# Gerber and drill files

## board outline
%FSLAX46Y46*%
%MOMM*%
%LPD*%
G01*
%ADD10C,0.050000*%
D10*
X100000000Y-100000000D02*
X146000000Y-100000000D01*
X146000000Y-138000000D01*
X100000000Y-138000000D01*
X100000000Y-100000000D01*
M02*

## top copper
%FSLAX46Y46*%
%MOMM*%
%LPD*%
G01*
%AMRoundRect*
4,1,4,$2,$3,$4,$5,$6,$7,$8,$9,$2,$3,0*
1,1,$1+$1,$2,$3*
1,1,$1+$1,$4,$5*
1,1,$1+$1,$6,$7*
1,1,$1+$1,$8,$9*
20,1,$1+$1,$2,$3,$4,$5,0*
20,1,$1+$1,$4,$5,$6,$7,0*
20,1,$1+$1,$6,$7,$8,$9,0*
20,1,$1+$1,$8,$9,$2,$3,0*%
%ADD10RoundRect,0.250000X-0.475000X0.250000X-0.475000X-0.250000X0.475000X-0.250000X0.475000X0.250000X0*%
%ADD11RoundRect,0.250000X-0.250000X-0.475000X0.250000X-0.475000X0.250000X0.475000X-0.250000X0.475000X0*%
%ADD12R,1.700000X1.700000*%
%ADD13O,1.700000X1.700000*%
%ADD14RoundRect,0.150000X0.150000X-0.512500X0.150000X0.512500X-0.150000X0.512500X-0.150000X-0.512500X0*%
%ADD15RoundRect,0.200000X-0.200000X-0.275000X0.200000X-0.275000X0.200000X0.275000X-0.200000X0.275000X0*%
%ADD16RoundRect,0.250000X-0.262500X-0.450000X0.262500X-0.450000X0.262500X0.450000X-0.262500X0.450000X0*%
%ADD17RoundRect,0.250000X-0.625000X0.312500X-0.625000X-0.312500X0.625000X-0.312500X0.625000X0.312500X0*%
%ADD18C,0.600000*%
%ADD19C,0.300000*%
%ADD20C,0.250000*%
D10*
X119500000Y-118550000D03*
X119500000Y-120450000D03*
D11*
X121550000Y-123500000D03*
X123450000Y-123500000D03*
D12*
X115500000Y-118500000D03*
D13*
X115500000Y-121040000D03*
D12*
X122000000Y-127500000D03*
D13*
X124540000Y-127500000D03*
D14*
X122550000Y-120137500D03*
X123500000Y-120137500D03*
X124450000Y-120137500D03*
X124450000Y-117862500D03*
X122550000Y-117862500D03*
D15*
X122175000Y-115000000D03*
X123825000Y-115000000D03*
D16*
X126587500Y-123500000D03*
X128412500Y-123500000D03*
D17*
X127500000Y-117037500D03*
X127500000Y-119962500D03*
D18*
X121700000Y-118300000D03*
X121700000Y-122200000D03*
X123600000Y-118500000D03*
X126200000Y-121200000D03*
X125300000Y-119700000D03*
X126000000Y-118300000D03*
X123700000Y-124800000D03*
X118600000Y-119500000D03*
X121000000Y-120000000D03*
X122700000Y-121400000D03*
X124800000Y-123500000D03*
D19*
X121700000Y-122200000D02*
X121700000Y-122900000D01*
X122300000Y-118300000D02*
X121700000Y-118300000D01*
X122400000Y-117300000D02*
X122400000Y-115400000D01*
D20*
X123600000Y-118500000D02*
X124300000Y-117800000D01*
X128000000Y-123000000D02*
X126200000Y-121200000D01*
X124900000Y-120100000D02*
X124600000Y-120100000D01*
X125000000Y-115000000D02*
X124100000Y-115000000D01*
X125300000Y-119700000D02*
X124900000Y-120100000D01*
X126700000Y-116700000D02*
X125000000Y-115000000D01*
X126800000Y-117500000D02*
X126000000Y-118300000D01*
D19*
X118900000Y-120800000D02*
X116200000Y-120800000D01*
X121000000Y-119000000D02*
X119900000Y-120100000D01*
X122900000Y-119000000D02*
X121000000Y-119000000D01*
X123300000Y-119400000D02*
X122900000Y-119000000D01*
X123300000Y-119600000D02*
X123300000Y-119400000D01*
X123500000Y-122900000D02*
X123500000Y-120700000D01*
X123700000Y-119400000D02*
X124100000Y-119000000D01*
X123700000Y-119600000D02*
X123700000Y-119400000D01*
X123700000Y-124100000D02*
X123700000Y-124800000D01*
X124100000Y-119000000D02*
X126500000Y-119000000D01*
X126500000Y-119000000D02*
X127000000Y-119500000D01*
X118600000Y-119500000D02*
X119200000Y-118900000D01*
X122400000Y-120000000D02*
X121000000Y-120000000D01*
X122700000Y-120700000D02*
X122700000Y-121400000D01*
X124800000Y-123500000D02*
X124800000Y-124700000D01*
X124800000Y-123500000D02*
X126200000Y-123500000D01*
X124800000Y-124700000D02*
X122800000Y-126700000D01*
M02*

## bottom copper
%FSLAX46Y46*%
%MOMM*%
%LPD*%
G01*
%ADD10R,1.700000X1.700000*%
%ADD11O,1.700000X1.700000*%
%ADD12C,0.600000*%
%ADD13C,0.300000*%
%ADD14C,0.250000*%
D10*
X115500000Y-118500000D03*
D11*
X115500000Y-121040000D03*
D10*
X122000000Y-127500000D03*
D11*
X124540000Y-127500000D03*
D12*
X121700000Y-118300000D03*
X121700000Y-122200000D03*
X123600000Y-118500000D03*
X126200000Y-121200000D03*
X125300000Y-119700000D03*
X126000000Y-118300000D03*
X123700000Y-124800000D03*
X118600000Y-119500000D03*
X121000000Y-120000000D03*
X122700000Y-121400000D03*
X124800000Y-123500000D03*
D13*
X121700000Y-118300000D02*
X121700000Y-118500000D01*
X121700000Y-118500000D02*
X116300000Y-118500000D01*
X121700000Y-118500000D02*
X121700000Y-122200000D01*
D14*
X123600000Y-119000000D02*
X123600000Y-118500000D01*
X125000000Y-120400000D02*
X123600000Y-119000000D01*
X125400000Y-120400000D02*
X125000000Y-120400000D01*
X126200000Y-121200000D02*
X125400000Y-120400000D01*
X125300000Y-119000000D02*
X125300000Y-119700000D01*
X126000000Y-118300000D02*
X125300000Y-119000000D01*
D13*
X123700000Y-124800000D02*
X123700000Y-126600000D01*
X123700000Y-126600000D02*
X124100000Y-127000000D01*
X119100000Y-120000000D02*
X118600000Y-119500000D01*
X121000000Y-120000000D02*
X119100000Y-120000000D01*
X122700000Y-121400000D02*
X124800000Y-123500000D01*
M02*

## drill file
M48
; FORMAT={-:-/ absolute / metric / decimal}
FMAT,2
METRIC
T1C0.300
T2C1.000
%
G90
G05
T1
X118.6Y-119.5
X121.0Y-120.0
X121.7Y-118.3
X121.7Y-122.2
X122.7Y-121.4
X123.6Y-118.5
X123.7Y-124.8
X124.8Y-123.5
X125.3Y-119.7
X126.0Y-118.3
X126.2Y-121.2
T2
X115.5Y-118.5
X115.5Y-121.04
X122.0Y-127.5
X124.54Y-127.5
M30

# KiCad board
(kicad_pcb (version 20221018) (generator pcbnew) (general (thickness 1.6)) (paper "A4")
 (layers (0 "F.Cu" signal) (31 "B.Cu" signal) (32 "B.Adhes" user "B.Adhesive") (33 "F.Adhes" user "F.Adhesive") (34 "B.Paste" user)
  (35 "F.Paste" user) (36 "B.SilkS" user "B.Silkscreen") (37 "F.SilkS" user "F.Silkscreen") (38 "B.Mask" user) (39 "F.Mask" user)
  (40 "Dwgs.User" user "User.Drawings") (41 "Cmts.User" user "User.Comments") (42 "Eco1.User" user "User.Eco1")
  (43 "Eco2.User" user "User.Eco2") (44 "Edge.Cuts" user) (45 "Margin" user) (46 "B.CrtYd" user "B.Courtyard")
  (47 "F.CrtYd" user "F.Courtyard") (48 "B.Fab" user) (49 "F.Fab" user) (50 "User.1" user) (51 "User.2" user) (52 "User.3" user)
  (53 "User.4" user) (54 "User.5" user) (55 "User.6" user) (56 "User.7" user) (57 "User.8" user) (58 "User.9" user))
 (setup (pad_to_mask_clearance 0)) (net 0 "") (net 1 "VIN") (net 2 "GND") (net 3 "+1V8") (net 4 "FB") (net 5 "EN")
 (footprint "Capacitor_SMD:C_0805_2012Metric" (layer "F.Cu") (at 119.5 119.5 -90)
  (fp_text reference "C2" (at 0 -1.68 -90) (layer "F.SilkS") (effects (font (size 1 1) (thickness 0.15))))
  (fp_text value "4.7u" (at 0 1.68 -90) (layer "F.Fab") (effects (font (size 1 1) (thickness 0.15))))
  (pad "1" smd roundrect (at -0.95 0 270) (size 1 1.45) (layers "F.Cu" "F.Paste" "F.Mask") (roundrect_rratio 0.25) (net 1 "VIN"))
  (pad "2" smd roundrect (at 0.95 0 270) (size 1 1.45) (layers "F.Cu" "F.Paste" "F.Mask") (roundrect_rratio 0.25) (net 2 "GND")))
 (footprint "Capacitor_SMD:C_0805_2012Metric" (layer "F.Cu") (at 122.5 123.5)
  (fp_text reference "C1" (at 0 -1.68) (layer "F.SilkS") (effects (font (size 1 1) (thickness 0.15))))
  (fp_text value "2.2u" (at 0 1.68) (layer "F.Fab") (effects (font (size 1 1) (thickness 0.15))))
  (pad "1" smd roundrect (at -0.95 0) (size 1 1.45) (layers "F.Cu" "F.Paste" "F.Mask") (roundrect_rratio 0.25) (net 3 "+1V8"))
  (pad "2" smd roundrect (at 0.95 0) (size 1 1.45) (layers "F.Cu" "F.Paste" "F.Mask") (roundrect_rratio 0.25) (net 2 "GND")))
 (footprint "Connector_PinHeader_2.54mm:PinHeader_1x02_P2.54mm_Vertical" (layer "F.Cu") (at 115.5 118.5)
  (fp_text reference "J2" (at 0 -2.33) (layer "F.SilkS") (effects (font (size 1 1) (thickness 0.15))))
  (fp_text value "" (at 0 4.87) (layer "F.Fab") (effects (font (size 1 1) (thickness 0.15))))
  (pad "1" thru_hole rect (at 0 0) (size 1.7 1.7) (drill 1) (layers "*.Cu" "*.Mask") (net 3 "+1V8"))
  (pad "2" thru_hole oval (at 0 2.54) (size 1.7 1.7) (drill 1) (layers "*.Cu" "*.Mask") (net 2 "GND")))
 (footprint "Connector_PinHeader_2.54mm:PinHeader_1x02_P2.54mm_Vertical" (layer "F.Cu") (at 122 127.5 90)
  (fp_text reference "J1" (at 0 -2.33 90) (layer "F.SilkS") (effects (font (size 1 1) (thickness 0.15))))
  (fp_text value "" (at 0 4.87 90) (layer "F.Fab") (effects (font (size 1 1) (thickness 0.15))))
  (pad "1" thru_hole rect (at 0 0 90) (size 1.7 1.7) (drill 1) (layers "*.Cu" "*.Mask") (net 1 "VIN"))
  (pad "2" thru_hole oval (at 0 2.54 90) (size 1.7 1.7) (drill 1) (layers "*.Cu" "*.Mask") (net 2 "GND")))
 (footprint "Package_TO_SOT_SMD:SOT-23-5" (layer "F.Cu") (at 123.5 119 90)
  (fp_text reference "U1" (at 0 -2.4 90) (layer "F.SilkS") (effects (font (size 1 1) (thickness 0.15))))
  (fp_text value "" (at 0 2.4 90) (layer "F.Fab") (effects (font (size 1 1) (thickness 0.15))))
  (pad "1" smd roundrect (at -1.1375 -0.95 90) (size 1.325 0.6) (layers "F.Cu" "F.Paste" "F.Mask") (roundrect_rratio 0.25) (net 1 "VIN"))
  (pad "2" smd roundrect (at -1.1375 0 90) (size 1.325 0.6) (layers "F.Cu" "F.Paste" "F.Mask") (roundrect_rratio 0.25) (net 2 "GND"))
  (pad "3" smd roundrect (at -1.1375 0.95 90) (size 1.325 0.6) (layers "F.Cu" "F.Paste" "F.Mask") (roundrect_rratio 0.25) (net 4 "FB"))
  (pad "4" smd roundrect (at 1.1375 0.95 90) (size 1.325 0.6) (layers "F.Cu" "F.Paste" "F.Mask") (roundrect_rratio 0.25) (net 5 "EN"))
  (pad "5" smd roundrect (at 1.1375 -0.95 90) (size 1.325 0.6) (layers "F.Cu" "F.Paste" "F.Mask") (roundrect_rratio 0.25) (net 3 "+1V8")))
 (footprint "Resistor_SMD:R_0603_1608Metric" (layer "F.Cu") (at 123 115)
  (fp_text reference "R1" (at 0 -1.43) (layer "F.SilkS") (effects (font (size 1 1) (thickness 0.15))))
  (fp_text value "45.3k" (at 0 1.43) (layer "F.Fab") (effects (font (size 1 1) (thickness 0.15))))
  (pad "1" smd roundrect (at -0.825 0) (size 0.8 0.95) (layers "F.Cu" "F.Paste" "F.Mask") (roundrect_rratio 0.25) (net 3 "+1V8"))
  (pad "2" smd roundrect (at 0.825 0) (size 0.8 0.95) (layers "F.Cu" "F.Paste" "F.Mask") (roundrect_rratio 0.25) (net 4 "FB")))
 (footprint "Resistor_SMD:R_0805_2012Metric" (layer "F.Cu") (at 127.5 123.5)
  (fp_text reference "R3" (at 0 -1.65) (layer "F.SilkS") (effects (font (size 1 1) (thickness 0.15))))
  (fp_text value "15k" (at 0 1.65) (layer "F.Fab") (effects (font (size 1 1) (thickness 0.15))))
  (pad "1" smd roundrect (at -0.9125 0) (size 1.025 1.4) (layers "F.Cu" "F.Paste" "F.Mask") (roundrect_rratio 0.243902) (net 1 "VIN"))
  (pad "2" smd roundrect (at 0.9125 0) (size 1.025 1.4) (layers "F.Cu" "F.Paste" "F.Mask") (roundrect_rratio 0.243902) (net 5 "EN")))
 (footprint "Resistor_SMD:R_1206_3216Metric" (layer "F.Cu") (at 127.5 118.5 -90)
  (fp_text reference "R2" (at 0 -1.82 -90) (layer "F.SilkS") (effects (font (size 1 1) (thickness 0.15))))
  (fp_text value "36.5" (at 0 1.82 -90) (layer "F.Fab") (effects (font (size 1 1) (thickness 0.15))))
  (pad "1" smd roundrect (at -1.4625 0 270) (size 1.125 1.75) (layers "F.Cu" "F.Paste" "F.Mask") (roundrect_rratio 0.222222) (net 4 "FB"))
  (pad "2" smd roundrect (at 1.4625 0 270) (size 1.125 1.75) (layers "F.Cu" "F.Paste" "F.Mask") (roundrect_rratio 0.222222) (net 2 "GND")))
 (gr_rect (start 100 100) (end 146 138) (stroke (width 0.05) (type default)) (fill none) (layer "Edge.Cuts"))
 (segment (start 121.7 122.2) (end 121.7 122.9) (width 0.3) (layer "F.Cu") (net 3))
 (segment (start 122.3 118.3) (end 121.7 118.3) (width 0.3) (layer "F.Cu") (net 3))
 (segment (start 122.4 117.3) (end 122.4 115.4) (width 0.3) (layer "F.Cu") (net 3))
 (via (at 121.7 118.3) (size 0.6) (drill 0.3) (layers "F.Cu" "B.Cu") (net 3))
 (via (at 121.7 122.2) (size 0.6) (drill 0.3) (layers "F.Cu" "B.Cu") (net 3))
 (segment (start 121.7 118.3) (end 121.7 118.5) (width 0.3) (layer "B.Cu") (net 3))
 (segment (start 121.7 118.5) (end 116.3 118.5) (width 0.3) (layer "B.Cu") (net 3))
 (segment (start 121.7 118.5) (end 121.7 122.2) (width 0.3) (layer "B.Cu") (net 3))
 (segment (start 123.6 118.5) (end 124.3 117.8) (width 0.25) (layer "F.Cu") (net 5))
 (segment (start 128 123) (end 126.2 121.2) (width 0.25) (layer "F.Cu") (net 5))
 (via (at 123.6 118.5) (size 0.6) (drill 0.3) (layers "F.Cu" "B.Cu") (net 5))
 (via (at 126.2 121.2) (size 0.6) (drill 0.3) (layers "F.Cu" "B.Cu") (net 5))
 (segment (start 123.6 119) (end 123.6 118.5) (width 0.25) (layer "B.Cu") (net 5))
 (segment (start 124.9 120.1) (end 124.6 120.1) (width 0.25) (layer "F.Cu") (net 4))
 (segment (start 125 115) (end 124.1 115) (width 0.25) (layer "F.Cu") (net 4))
 (segment (start 125 120.4) (end 123.6 119) (width 0.25) (layer "B.Cu") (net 5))
 (segment (start 125.3 119.7) (end 124.9 120.1) (width 0.25) (layer "F.Cu") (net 4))
 (segment (start 125.4 120.4) (end 125 120.4) (width 0.25) (layer "B.Cu") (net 5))
 (segment (start 126.2 121.2) (end 125.4 120.4) (width 0.25) (layer "B.Cu") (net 5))
 (segment (start 126.7 116.7) (end 125 115) (width 0.25) (layer "F.Cu") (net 4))
 (segment (start 126.8 117.5) (end 126 118.3) (width 0.25) (layer "F.Cu") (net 4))
 (via (at 125.3 119.7) (size 0.6) (drill 0.3) (layers "F.Cu" "B.Cu") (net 4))
 (via (at 126 118.3) (size 0.6) (drill 0.3) (layers "F.Cu" "B.Cu") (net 4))
 (segment (start 118.9 120.8) (end 116.2 120.8) (width 0.3) (layer "F.Cu") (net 2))
 (segment (start 121 119) (end 119.9 120.1) (width 0.3) (layer "F.Cu") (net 2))
 (segment (start 122.9 119) (end 121 119) (width 0.3) (layer "F.Cu") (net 2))
 (segment (start 123.3 119.4) (end 122.9 119) (width 0.3) (layer "F.Cu") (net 2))
 (segment (start 123.3 119.6) (end 123.3 119.4) (width 0.3) (layer "F.Cu") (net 2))
 (segment (start 123.5 122.9) (end 123.5 120.7) (width 0.3) (layer "F.Cu") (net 2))
 (segment (start 123.7 119.4) (end 124.1 119) (width 0.3) (layer "F.Cu") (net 2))
 (segment (start 123.7 119.6) (end 123.7 119.4) (width 0.3) (layer "F.Cu") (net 2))
 (segment (start 123.7 124.1) (end 123.7 124.8) (width 0.3) (layer "F.Cu") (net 2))
 (segment (start 124.1 119) (end 126.5 119) (width 0.3) (layer "F.Cu") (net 2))
 (segment (start 125.3 119) (end 125.3 119.7) (width 0.25) (layer "B.Cu") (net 4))
 (segment (start 126 118.3) (end 125.3 119) (width 0.25) (layer "B.Cu") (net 4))
 (segment (start 126.5 119) (end 127 119.5) (width 0.3) (layer "F.Cu") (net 2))
 (via (at 123.7 124.8) (size 0.6) (drill 0.3) (layers "F.Cu" "B.Cu") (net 2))
 (segment (start 118.6 119.5) (end 119.2 118.9) (width 0.3) (layer "F.Cu") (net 1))
 (segment (start 122.4 120) (end 121 120) (width 0.3) (layer "F.Cu") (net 1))
 (segment (start 122.7 120.7) (end 122.7 121.4) (width 0.3) (layer "F.Cu") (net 1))
 (segment (start 123.7 124.8) (end 123.7 126.6) (width 0.3) (layer "B.Cu") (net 2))
 (segment (start 123.7 126.6) (end 124.1 127) (width 0.3) (layer "B.Cu") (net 2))
 (segment (start 124.8 123.5) (end 124.8 124.7) (width 0.3) (layer "F.Cu") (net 1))
 (segment (start 124.8 123.5) (end 126.2 123.5) (width 0.3) (layer "F.Cu") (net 1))
 (segment (start 124.8 124.7) (end 122.8 126.7) (width 0.3) (layer "F.Cu") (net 1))
 (via (at 118.6 119.5) (size 0.6) (drill 0.3) (layers "F.Cu" "B.Cu") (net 1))
 (via (at 121 120) (size 0.6) (drill 0.3) (layers "F.Cu" "B.Cu") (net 1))
 (via (at 122.7 121.4) (size 0.6) (drill 0.3) (layers "F.Cu" "B.Cu") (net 1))
 (via (at 124.8 123.5) (size 0.6) (drill 0.3) (layers "F.Cu" "B.Cu") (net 1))
 (segment (start 119.1 120) (end 118.6 119.5) (width 0.3) (layer "B.Cu") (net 1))
 (segment (start 121 120) (end 119.1 120) (width 0.3) (layer "B.Cu") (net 1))
 (segment (start 122.7 121.4) (end 124.8 123.5) (width 0.3) (layer "B.Cu") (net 1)))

